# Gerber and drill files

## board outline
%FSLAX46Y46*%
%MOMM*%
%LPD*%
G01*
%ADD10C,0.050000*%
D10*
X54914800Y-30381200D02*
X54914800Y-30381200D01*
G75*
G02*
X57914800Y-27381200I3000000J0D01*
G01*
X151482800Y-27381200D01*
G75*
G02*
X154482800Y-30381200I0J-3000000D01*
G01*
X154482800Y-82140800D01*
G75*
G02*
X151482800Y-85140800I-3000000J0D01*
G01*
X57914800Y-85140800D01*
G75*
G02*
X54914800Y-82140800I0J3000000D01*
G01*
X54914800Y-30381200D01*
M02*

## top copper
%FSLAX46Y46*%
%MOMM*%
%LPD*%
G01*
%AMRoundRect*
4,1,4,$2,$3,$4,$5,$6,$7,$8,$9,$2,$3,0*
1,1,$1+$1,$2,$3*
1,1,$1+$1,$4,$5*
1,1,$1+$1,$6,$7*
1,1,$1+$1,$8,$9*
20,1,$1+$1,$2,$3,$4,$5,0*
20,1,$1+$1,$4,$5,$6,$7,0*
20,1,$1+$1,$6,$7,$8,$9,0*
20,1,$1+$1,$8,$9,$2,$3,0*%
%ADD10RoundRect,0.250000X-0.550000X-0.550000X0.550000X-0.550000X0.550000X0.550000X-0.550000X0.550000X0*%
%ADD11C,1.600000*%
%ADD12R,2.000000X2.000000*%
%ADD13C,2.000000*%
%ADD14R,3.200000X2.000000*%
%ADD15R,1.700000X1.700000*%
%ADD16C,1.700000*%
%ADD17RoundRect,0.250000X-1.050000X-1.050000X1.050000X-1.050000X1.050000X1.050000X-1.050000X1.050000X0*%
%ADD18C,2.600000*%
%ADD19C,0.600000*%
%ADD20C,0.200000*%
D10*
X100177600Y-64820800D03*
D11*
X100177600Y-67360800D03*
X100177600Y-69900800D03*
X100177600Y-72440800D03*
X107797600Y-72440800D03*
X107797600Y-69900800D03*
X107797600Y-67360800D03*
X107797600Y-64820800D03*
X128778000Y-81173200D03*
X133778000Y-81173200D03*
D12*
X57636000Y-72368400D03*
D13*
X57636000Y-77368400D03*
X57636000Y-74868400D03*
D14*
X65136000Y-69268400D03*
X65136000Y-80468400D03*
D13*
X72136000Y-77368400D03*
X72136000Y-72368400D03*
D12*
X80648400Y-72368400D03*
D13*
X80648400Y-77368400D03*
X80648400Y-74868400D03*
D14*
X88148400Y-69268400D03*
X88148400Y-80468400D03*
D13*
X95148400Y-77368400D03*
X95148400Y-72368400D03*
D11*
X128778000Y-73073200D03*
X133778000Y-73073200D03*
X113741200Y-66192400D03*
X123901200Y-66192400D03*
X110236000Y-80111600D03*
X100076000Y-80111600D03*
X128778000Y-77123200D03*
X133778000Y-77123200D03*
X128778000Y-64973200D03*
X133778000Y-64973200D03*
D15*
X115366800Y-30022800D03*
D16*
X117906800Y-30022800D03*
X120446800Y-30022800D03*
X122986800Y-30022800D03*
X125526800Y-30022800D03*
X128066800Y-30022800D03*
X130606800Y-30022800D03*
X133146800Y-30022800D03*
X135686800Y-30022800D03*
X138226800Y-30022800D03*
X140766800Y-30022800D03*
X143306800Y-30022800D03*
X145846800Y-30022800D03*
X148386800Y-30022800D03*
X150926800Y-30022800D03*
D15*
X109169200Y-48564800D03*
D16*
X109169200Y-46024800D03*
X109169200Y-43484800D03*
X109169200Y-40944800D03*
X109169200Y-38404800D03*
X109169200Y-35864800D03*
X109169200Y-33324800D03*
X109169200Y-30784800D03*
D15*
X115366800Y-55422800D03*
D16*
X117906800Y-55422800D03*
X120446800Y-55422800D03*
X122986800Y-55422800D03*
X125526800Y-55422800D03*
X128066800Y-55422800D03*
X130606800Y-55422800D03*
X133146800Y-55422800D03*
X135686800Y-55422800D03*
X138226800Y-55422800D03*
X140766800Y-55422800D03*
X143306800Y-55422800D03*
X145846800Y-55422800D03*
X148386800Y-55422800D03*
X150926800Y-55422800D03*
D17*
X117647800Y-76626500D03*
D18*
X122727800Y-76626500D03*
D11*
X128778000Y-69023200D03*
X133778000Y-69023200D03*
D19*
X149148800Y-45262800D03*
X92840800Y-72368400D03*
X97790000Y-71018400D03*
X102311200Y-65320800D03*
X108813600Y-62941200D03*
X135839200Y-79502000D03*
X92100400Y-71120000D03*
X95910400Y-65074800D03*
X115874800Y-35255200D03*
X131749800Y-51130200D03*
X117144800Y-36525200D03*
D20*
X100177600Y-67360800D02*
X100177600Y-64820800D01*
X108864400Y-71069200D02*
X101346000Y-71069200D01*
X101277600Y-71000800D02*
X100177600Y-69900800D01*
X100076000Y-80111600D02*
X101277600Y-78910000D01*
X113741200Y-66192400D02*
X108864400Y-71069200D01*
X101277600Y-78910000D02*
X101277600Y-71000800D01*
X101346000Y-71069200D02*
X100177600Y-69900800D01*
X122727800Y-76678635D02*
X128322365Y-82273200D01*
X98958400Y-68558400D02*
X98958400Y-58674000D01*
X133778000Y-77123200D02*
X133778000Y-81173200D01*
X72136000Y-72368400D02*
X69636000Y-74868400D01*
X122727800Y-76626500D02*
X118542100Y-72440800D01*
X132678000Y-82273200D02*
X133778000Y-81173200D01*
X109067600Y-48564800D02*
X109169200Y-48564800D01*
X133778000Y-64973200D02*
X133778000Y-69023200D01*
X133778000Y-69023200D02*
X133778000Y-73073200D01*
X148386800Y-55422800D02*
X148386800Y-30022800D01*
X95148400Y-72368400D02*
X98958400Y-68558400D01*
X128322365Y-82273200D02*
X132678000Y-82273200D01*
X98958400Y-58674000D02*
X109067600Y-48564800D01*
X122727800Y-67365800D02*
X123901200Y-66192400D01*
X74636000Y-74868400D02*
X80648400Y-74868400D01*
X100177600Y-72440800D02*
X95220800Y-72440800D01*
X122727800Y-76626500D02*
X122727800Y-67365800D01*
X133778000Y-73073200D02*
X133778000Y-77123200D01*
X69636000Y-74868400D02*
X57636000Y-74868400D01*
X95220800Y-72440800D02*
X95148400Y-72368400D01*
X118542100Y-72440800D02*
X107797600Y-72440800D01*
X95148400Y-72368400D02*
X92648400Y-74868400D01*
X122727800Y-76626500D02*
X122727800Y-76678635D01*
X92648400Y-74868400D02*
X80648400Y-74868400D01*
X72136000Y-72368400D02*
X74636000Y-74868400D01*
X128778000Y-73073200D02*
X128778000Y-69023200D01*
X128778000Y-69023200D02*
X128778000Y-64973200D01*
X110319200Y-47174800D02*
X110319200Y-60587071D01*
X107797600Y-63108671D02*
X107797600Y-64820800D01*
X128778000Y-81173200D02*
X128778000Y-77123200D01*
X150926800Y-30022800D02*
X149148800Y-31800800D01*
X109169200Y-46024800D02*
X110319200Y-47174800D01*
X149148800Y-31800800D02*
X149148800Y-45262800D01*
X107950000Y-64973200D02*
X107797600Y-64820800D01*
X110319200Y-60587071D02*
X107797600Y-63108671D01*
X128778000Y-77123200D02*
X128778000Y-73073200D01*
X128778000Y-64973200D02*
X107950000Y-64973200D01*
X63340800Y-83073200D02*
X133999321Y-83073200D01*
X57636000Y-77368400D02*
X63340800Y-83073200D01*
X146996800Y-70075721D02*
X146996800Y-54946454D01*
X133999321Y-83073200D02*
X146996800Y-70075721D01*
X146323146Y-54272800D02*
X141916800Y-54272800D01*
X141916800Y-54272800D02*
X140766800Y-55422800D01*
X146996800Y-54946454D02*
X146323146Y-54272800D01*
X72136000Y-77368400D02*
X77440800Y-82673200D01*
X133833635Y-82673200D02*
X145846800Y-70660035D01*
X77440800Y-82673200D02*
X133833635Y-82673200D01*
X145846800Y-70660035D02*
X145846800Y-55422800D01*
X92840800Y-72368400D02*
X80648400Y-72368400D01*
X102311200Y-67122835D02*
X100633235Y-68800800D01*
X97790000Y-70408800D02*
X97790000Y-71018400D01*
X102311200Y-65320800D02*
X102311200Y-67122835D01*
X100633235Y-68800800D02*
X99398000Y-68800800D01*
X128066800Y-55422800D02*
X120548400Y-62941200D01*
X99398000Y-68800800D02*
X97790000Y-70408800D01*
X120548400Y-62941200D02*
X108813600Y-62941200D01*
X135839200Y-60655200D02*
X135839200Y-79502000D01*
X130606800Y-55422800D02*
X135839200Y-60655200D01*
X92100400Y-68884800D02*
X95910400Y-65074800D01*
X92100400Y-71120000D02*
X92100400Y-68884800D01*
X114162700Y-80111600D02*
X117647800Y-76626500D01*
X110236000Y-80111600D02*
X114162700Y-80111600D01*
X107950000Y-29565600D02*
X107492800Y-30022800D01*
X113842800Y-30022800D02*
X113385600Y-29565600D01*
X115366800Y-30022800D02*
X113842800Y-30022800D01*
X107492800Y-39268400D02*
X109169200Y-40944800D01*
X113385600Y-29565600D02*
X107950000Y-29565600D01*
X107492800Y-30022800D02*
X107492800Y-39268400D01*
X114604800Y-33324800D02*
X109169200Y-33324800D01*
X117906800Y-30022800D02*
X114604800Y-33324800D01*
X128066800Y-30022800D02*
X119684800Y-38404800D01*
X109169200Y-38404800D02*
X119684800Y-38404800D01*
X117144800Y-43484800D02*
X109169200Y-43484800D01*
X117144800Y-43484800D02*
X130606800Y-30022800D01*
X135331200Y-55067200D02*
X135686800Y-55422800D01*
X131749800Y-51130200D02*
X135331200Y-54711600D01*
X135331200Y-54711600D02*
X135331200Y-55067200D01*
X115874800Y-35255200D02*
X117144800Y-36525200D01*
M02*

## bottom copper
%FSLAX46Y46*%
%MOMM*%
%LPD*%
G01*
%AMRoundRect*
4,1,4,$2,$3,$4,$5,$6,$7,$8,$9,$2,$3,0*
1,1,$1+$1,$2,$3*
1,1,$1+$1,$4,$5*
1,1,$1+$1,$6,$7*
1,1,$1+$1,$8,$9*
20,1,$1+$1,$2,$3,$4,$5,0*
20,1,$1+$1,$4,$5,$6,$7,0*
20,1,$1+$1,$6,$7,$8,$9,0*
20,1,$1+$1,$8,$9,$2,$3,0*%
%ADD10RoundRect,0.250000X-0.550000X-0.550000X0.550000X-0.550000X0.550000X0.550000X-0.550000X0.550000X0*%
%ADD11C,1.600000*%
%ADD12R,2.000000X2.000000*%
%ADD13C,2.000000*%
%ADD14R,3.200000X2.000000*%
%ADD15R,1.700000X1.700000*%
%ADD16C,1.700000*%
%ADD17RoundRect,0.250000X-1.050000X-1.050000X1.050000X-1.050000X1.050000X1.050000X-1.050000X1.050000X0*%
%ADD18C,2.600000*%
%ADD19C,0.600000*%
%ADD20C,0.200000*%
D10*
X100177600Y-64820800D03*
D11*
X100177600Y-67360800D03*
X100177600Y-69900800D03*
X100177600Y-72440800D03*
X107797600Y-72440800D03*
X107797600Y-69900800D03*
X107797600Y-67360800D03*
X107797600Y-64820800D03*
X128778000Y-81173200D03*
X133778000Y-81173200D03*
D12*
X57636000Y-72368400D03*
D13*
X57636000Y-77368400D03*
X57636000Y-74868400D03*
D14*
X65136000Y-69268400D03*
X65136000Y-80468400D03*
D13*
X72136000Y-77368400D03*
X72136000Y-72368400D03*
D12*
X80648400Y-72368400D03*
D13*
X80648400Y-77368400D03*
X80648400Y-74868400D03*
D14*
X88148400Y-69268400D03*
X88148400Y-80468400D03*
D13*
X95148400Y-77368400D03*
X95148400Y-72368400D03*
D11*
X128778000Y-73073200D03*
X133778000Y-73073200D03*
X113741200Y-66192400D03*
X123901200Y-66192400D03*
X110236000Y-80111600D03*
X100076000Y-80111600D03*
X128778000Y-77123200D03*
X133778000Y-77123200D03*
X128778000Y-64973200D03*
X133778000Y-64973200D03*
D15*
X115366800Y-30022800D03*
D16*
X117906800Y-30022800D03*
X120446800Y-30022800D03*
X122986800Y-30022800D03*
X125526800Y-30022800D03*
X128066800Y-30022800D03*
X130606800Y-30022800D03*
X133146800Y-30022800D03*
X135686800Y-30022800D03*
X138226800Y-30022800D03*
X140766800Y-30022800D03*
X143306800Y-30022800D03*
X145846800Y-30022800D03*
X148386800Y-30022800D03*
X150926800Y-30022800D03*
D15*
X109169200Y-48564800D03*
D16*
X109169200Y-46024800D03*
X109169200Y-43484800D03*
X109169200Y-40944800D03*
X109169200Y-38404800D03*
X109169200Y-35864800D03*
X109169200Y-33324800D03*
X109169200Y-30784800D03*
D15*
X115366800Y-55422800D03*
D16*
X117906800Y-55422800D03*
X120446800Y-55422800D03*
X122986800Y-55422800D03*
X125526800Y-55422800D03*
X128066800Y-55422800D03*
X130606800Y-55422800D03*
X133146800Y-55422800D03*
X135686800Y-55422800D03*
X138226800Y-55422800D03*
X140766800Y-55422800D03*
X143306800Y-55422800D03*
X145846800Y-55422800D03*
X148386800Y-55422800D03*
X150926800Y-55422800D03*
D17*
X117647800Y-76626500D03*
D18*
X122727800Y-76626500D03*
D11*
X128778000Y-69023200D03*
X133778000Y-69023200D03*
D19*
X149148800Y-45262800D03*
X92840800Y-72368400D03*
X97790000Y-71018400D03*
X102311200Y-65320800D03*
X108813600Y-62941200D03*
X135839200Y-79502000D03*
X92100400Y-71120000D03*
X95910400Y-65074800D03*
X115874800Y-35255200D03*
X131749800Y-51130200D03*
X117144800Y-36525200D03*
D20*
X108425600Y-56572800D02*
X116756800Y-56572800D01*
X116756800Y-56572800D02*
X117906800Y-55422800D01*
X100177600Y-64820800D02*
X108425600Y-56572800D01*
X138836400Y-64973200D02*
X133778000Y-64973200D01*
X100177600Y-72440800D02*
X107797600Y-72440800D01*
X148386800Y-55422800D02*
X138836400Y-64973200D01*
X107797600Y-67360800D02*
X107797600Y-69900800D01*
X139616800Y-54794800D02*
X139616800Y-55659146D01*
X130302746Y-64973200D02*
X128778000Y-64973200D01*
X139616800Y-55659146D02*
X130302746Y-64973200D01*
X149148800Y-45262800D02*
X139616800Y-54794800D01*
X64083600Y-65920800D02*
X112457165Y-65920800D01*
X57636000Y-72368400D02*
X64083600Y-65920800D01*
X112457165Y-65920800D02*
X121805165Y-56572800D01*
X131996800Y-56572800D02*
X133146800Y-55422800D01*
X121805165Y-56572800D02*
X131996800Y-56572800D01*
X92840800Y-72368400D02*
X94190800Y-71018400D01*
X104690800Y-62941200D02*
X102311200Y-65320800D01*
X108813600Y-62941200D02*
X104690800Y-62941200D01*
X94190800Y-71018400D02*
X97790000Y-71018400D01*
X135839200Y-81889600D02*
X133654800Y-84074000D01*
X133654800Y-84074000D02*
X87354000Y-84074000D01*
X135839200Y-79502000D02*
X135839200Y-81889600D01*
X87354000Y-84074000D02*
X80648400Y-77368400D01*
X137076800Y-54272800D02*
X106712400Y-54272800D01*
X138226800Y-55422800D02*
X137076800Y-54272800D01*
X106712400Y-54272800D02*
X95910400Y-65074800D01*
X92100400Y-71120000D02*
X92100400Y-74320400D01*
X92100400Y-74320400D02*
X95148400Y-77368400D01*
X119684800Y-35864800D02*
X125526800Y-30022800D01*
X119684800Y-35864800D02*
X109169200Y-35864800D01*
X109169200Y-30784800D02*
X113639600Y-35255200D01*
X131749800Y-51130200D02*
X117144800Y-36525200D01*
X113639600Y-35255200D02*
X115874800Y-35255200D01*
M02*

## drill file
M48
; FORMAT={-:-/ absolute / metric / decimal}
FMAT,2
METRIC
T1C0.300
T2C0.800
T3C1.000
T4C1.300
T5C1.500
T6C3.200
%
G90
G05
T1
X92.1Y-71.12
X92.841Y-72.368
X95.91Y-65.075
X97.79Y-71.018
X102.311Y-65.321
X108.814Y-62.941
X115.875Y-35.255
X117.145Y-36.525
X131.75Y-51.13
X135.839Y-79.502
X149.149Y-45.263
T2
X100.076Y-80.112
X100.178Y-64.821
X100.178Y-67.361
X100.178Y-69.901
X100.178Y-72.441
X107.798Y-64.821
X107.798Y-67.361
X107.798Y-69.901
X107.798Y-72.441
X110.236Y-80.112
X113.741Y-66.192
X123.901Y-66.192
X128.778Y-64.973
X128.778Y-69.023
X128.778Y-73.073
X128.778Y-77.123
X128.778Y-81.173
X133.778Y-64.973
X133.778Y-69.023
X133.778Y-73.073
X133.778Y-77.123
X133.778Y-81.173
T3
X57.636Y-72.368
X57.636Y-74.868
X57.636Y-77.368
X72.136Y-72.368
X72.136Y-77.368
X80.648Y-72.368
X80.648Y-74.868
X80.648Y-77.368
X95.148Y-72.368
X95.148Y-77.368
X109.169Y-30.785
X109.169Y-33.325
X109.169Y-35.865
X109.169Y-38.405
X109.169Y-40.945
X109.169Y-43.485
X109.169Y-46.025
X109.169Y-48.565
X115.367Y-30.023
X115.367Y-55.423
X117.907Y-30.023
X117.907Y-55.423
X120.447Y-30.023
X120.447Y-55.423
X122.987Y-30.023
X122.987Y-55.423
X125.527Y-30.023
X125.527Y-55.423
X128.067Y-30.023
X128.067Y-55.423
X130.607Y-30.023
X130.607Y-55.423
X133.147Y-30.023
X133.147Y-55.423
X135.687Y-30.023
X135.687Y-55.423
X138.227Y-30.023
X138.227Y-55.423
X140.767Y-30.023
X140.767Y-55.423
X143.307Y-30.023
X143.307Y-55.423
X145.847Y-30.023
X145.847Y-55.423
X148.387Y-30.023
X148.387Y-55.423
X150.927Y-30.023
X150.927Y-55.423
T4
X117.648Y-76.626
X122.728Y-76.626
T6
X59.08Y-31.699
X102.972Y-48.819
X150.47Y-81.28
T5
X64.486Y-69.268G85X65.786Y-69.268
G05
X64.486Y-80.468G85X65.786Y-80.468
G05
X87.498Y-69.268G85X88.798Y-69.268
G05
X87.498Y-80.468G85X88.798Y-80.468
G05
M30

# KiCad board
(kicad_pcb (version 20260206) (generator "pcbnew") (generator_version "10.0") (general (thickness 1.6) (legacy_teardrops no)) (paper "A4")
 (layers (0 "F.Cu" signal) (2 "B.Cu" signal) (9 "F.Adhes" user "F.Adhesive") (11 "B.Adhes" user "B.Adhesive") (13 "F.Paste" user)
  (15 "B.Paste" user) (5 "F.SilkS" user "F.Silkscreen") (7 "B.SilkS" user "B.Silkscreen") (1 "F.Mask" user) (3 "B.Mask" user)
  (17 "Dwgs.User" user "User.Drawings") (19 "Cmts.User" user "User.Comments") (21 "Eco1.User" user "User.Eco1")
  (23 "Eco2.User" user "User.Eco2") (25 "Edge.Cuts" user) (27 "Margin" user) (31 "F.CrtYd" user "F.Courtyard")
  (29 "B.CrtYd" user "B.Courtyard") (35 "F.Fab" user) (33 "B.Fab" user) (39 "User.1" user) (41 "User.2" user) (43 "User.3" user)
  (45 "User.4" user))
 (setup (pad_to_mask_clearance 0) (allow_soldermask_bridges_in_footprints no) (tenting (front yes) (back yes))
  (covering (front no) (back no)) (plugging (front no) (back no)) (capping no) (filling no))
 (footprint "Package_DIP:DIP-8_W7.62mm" (layer "F.Cu") (at 100.1776 64.8208)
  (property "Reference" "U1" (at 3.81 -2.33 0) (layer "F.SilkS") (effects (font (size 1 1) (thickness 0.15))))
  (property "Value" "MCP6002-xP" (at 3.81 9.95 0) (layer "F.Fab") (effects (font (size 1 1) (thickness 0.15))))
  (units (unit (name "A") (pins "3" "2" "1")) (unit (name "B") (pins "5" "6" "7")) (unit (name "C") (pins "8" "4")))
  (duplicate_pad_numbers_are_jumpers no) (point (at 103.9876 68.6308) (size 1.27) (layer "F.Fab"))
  (pad "1" thru_hole roundrect (at 0 0) (size 1.6 1.6) (drill 0.8) (layers "*.Cu" "*.Mask") (remove_unused_layers no)
   (roundrect_rratio 0.15625) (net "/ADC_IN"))
  (pad "2" thru_hole circle (at 0 2.54) (size 1.6 1.6) (drill 0.8) (layers "*.Cu" "*.Mask") (remove_unused_layers no) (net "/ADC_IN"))
  (pad "3" thru_hole circle (at 0 5.08) (size 1.6 1.6) (drill 0.8) (layers "*.Cu" "*.Mask") (remove_unused_layers no) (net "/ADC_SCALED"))
  (pad "4" thru_hole circle (at 0 7.62) (size 1.6 1.6) (drill 0.8) (layers "*.Cu" "*.Mask") (remove_unused_layers no) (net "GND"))
  (pad "5" thru_hole circle (at 7.62 7.62) (size 1.6 1.6) (drill 0.8) (layers "*.Cu" "*.Mask") (remove_unused_layers no) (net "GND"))
  (pad "6" thru_hole circle (at 7.62 5.08) (size 1.6 1.6) (drill 0.8) (layers "*.Cu" "*.Mask") (remove_unused_layers no) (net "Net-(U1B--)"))
  (pad "7" thru_hole circle (at 7.62 2.54) (size 1.6 1.6) (drill 0.8) (layers "*.Cu" "*.Mask") (remove_unused_layers no) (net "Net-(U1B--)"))
  (pad "8" thru_hole circle (at 7.62 0) (size 1.6 1.6) (drill 0.8) (layers "*.Cu" "*.Mask") (remove_unused_layers no) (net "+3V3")))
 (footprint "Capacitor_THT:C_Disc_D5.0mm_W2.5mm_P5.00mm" (layer "F.Cu") (at 128.778 81.1732)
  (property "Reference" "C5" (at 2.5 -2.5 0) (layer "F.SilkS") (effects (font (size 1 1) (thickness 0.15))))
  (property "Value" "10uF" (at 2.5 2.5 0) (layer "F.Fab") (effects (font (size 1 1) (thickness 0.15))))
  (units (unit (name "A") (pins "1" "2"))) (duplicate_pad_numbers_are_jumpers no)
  (pad "1" thru_hole circle (at 0 0) (size 1.6 1.6) (drill 0.8) (layers "*.Cu" "*.Mask") (remove_unused_layers no) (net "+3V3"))
  (pad "2" thru_hole circle (at 5 0) (size 1.6 1.6) (drill 0.8) (layers "*.Cu" "*.Mask") (remove_unused_layers no) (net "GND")))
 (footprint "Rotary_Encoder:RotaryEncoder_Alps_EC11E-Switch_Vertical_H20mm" (layer "F.Cu") (at 57.636 72.3684)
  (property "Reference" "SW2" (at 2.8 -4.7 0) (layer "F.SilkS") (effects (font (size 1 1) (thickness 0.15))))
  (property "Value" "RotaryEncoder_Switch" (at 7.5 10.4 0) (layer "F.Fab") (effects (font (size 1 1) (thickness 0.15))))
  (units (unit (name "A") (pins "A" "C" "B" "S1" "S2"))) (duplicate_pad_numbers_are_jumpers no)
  (pad "A" thru_hole rect (at 0 0) (size 2 2) (drill 1) (layers "*.Cu" "*.Mask") (remove_unused_layers no) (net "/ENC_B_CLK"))
  (pad "B" thru_hole circle (at 0 5) (size 2 2) (drill 1) (layers "*.Cu" "*.Mask") (remove_unused_layers no) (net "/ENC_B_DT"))
  (pad "C" thru_hole circle (at 0 2.5) (size 2 2) (drill 1) (layers "*.Cu" "*.Mask") (remove_unused_layers no) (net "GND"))
  (pad "MP" thru_hole rect (at 7.5 -3.1) (size 3.2 2) (drill oval 2.8 1.5) (layers "*.Cu" "*.Mask") (remove_unused_layers no))
  (pad "MP" thru_hole rect (at 7.5 8.1) (size 3.2 2) (drill oval 2.8 1.5) (layers "*.Cu" "*.Mask") (remove_unused_layers no))
  (pad "S1" thru_hole circle (at 14.5 5) (size 2 2) (drill 1) (layers "*.Cu" "*.Mask") (remove_unused_layers no) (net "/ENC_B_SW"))
  (pad "S2" thru_hole circle (at 14.5 0) (size 2 2) (drill 1) (layers "*.Cu" "*.Mask") (remove_unused_layers no) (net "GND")))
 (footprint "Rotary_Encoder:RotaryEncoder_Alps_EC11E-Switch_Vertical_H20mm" (layer "F.Cu") (at 80.6484 72.3684)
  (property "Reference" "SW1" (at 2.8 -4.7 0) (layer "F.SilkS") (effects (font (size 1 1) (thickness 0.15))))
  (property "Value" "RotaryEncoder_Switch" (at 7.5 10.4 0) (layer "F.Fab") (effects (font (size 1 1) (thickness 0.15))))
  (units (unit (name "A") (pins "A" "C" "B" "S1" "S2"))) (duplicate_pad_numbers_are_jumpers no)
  (pad "A" thru_hole rect (at 0 0) (size 2 2) (drill 1) (layers "*.Cu" "*.Mask") (remove_unused_layers no) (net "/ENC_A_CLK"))
  (pad "B" thru_hole circle (at 0 5) (size 2 2) (drill 1) (layers "*.Cu" "*.Mask") (remove_unused_layers no) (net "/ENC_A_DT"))
  (pad "C" thru_hole circle (at 0 2.5) (size 2 2) (drill 1) (layers "*.Cu" "*.Mask") (remove_unused_layers no) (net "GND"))
  (pad "MP" thru_hole rect (at 7.5 -3.1) (size 3.2 2) (drill oval 2.8 1.5) (layers "*.Cu" "*.Mask") (remove_unused_layers no))
  (pad "MP" thru_hole rect (at 7.5 8.1) (size 3.2 2) (drill oval 2.8 1.5) (layers "*.Cu" "*.Mask") (remove_unused_layers no))
  (pad "S1" thru_hole circle (at 14.5 5) (size 2 2) (drill 1) (layers "*.Cu" "*.Mask") (remove_unused_layers no) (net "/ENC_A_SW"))
  (pad "S2" thru_hole circle (at 14.5 0) (size 2 2) (drill 1) (layers "*.Cu" "*.Mask") (remove_unused_layers no) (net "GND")))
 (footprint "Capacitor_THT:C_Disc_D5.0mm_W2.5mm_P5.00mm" (layer "F.Cu") (at 128.778 73.0732)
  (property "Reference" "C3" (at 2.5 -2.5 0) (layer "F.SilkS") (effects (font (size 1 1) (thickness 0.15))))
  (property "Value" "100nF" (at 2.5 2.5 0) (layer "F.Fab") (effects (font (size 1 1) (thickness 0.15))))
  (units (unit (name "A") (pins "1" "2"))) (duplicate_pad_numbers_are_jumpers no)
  (pad "1" thru_hole circle (at 0 0) (size 1.6 1.6) (drill 0.8) (layers "*.Cu" "*.Mask") (remove_unused_layers no) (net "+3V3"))
  (pad "2" thru_hole circle (at 5 0) (size 1.6 1.6) (drill 0.8) (layers "*.Cu" "*.Mask") (remove_unused_layers no) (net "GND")))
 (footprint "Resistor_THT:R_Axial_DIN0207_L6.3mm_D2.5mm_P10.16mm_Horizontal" (layer "F.Cu") (at 113.7412 66.1924)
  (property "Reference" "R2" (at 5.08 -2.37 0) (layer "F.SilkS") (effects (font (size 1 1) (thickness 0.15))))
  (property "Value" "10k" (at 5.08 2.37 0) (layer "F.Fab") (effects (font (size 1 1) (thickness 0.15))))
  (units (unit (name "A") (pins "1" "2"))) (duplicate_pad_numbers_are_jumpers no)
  (pad "1" thru_hole circle (at 0 0) (size 1.6 1.6) (drill 0.8) (layers "*.Cu" "*.Mask") (remove_unused_layers no) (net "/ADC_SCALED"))
  (pad "2" thru_hole circle (at 10.16 0) (size 1.6 1.6) (drill 0.8) (layers "*.Cu" "*.Mask") (remove_unused_layers no) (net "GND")))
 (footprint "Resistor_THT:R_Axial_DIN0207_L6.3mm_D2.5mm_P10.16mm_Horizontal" (layer "F.Cu") (at 110.236 80.1116 180)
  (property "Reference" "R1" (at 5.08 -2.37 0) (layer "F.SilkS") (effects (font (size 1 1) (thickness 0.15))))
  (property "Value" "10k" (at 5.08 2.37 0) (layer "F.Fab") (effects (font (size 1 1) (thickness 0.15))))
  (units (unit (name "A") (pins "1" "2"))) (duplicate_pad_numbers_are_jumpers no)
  (pad "1" thru_hole circle (at 0 0 180) (size 1.6 1.6) (drill 0.8) (layers "*.Cu" "*.Mask") (remove_unused_layers no) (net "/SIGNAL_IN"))
  (pad "2" thru_hole circle (at 10.16 0 180) (size 1.6 1.6) (drill 0.8) (layers "*.Cu" "*.Mask") (remove_unused_layers no)
   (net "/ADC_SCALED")))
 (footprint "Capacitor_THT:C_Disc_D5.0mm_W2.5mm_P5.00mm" (layer "F.Cu") (at 128.778 77.1232)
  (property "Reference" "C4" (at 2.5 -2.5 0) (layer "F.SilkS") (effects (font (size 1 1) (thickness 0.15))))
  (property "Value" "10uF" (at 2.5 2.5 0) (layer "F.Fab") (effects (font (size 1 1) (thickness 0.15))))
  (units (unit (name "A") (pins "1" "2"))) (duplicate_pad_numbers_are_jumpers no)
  (pad "1" thru_hole circle (at 0 0) (size 1.6 1.6) (drill 0.8) (layers "*.Cu" "*.Mask") (remove_unused_layers no) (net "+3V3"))
  (pad "2" thru_hole circle (at 5 0) (size 1.6 1.6) (drill 0.8) (layers "*.Cu" "*.Mask") (remove_unused_layers no) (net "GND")))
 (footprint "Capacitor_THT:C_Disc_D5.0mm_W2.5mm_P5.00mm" (layer "F.Cu") (at 128.778 64.9732)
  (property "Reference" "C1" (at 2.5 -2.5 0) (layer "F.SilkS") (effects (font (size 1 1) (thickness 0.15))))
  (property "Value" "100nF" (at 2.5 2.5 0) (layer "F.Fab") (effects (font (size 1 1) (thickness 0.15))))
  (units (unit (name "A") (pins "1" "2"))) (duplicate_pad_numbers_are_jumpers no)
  (pad "1" thru_hole circle (at 0 0) (size 1.6 1.6) (drill 0.8) (layers "*.Cu" "*.Mask") (remove_unused_layers no) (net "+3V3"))
  (pad "2" thru_hole circle (at 5 0) (size 1.6 1.6) (drill 0.8) (layers "*.Cu" "*.Mask") (remove_unused_layers no) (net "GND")))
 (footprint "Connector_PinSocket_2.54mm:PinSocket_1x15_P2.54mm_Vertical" (layer "F.Cu") (at 115.3668 30.0228 90)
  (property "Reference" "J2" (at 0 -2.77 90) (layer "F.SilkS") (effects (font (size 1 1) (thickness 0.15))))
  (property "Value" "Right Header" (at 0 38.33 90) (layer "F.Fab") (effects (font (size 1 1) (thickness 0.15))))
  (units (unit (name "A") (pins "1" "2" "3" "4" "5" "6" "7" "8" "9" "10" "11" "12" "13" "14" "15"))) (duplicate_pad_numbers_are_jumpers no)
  (pad "1" thru_hole rect (at 0 0 90) (size 1.7 1.7) (drill 1) (layers "*.Cu" "*.Mask") (remove_unused_layers no) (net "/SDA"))
  (pad "2" thru_hole circle (at 0 2.54 90) (size 1.7 1.7) (drill 1) (layers "*.Cu" "*.Mask") (remove_unused_layers no) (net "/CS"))
  (pad "3" thru_hole circle (at 0 5.08 90) (size 1.7 1.7) (drill 1) (layers "*.Cu" "*.Mask") (remove_unused_layers no) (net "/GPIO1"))
  (pad "4" thru_hole circle (at 0 7.62 90) (size 1.7 1.7) (drill 1) (layers "*.Cu" "*.Mask") (remove_unused_layers no) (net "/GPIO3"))
  (pad "5" thru_hole circle (at 0 10.16 90) (size 1.7 1.7) (drill 1) (layers "*.Cu" "*.Mask") (remove_unused_layers no) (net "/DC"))
  (pad "6" thru_hole circle (at 0 12.7 90) (size 1.7 1.7) (drill 1) (layers "*.Cu" "*.Mask") (remove_unused_layers no) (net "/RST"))
  (pad "7" thru_hole circle (at 0 15.24 90) (size 1.7 1.7) (drill 1) (layers "*.Cu" "*.Mask") (remove_unused_layers no) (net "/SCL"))
  (pad "8" thru_hole circle (at 0 17.78 90) (size 1.7 1.7) (drill 1) (layers "*.Cu" "*.Mask") (remove_unused_layers no) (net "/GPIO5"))
  (pad "9" thru_hole circle (at 0 20.32 90) (size 1.7 1.7) (drill 1) (layers "*.Cu" "*.Mask") (remove_unused_layers no) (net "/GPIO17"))
  (pad "10" thru_hole circle (at 0 22.86 90) (size 1.7 1.7) (drill 1) (layers "*.Cu" "*.Mask") (remove_unused_layers no) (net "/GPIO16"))
  (pad "11" thru_hole circle (at 0 25.4 90) (size 1.7 1.7) (drill 1) (layers "*.Cu" "*.Mask") (remove_unused_layers no) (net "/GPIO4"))
  (pad "12" thru_hole circle (at 0 27.94 90) (size 1.7 1.7) (drill 1) (layers "*.Cu" "*.Mask") (remove_unused_layers no) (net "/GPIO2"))
  (pad "13" thru_hole circle (at 0 30.48 90) (size 1.7 1.7) (drill 1) (layers "*.Cu" "*.Mask") (remove_unused_layers no) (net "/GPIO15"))
  (pad "14" thru_hole circle (at 0 33.02 90) (size 1.7 1.7) (drill 1) (layers "*.Cu" "*.Mask") (remove_unused_layers no) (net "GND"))
  (pad "15" thru_hole circle (at 0 35.56 90) (size 1.7 1.7) (drill 1) (layers "*.Cu" "*.Mask") (remove_unused_layers no) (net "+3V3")))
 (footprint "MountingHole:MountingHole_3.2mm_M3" (layer "F.Cu") (at 150.4696 81.28)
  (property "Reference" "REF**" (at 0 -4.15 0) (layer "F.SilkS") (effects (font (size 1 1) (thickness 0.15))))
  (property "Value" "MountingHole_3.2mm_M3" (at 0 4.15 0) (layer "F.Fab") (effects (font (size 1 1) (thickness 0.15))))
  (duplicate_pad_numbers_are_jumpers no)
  (pad "" np_thru_hole circle (at 0 0) (size 3.2 3.2) (drill 3.2) (layers "*.Cu" "*.Mask")))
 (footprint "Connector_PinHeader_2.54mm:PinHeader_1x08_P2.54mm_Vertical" (layer "F.Cu") (at 109.1692 48.5648 180)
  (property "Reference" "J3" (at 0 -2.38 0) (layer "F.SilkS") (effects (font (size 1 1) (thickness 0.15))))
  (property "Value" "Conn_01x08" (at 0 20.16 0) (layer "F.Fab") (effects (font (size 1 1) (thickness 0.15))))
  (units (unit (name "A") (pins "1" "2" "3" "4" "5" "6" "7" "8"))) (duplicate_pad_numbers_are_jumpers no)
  (pad "1" thru_hole rect (at 0 0 180) (size 1.7 1.7) (drill 1) (layers "*.Cu" "*.Mask") (remove_unused_layers no) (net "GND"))
  (pad "2" thru_hole circle (at 0 2.54 180) (size 1.7 1.7) (drill 1) (layers "*.Cu" "*.Mask") (remove_unused_layers no) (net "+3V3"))
  (pad "3" thru_hole circle (at 0 5.08 180) (size 1.7 1.7) (drill 1) (layers "*.Cu" "*.Mask") (remove_unused_layers no) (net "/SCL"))
  (pad "4" thru_hole circle (at 0 7.62 180) (size 1.7 1.7) (drill 1) (layers "*.Cu" "*.Mask") (remove_unused_layers no) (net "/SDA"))
  (pad "5" thru_hole circle (at 0 10.16 180) (size 1.7 1.7) (drill 1) (layers "*.Cu" "*.Mask") (remove_unused_layers no) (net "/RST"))
  (pad "6" thru_hole circle (at 0 12.7 180) (size 1.7 1.7) (drill 1) (layers "*.Cu" "*.Mask") (remove_unused_layers no) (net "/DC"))
  (pad "7" thru_hole circle (at 0 15.24 180) (size 1.7 1.7) (drill 1) (layers "*.Cu" "*.Mask") (remove_unused_layers no) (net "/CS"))
  (pad "8" thru_hole circle (at 0 17.78 180) (size 1.7 1.7) (drill 1) (layers "*.Cu" "*.Mask") (remove_unused_layers no) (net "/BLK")))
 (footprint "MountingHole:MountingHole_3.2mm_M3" (layer "F.Cu") (at 102.9716 48.8188)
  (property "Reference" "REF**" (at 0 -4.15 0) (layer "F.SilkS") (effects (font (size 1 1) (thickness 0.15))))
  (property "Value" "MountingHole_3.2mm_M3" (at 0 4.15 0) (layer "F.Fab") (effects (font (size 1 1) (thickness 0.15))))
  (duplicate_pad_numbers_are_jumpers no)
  (pad "" np_thru_hole circle (at 0 0) (size 3.2 3.2) (drill 3.2) (layers "*.Cu" "*.Mask")))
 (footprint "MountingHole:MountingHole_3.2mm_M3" (layer "F.Cu") (at 59.0804 31.6992)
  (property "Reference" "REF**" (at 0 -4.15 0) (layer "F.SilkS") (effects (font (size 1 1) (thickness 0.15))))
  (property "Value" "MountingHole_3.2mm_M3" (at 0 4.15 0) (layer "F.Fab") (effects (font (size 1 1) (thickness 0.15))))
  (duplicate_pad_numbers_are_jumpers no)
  (pad "" np_thru_hole circle (at 0 0) (size 3.2 3.2) (drill 3.2) (layers "*.Cu" "*.Mask")))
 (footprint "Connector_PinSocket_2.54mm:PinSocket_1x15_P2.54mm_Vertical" (layer "F.Cu") (at 115.3668 55.4228 90)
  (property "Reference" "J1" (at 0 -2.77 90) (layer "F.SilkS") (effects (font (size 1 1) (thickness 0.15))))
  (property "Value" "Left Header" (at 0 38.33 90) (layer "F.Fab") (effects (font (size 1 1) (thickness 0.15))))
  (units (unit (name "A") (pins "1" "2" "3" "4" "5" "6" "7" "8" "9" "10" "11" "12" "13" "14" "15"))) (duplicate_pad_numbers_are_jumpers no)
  (pad "1" thru_hole rect (at 0 0 90) (size 1.7 1.7) (drill 1) (layers "*.Cu" "*.Mask") (remove_unused_layers no) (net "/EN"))
  (pad "2" thru_hole circle (at 0 2.54 90) (size 1.7 1.7) (drill 1) (layers "*.Cu" "*.Mask") (remove_unused_layers no) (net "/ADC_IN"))
  (pad "3" thru_hole circle (at 0 5.08 90) (size 1.7 1.7) (drill 1) (layers "*.Cu" "*.Mask") (remove_unused_layers no) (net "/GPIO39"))
  (pad "4" thru_hole circle (at 0 7.62 90) (size 1.7 1.7) (drill 1) (layers "*.Cu" "*.Mask") (remove_unused_layers no) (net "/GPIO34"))
  (pad "5" thru_hole circle (at 0 10.16 90) (size 1.7 1.7) (drill 1) (layers "*.Cu" "*.Mask") (remove_unused_layers no) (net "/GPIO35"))
  (pad "6" thru_hole circle (at 0 12.7 90) (size 1.7 1.7) (drill 1) (layers "*.Cu" "*.Mask") (remove_unused_layers no) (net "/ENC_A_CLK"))
  (pad "7" thru_hole circle (at 0 15.24 90) (size 1.7 1.7) (drill 1) (layers "*.Cu" "*.Mask") (remove_unused_layers no) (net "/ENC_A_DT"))
  (pad "8" thru_hole circle (at 0 17.78 90) (size 1.7 1.7) (drill 1) (layers "*.Cu" "*.Mask") (remove_unused_layers no) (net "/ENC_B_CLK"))
  (pad "9" thru_hole circle (at 0 20.32 90) (size 1.7 1.7) (drill 1) (layers "*.Cu" "*.Mask") (remove_unused_layers no) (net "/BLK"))
  (pad "10" thru_hole circle (at 0 22.86 90) (size 1.7 1.7) (drill 1) (layers "*.Cu" "*.Mask") (remove_unused_layers no) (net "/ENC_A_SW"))
  (pad "11" thru_hole circle (at 0 25.4 90) (size 1.7 1.7) (drill 1) (layers "*.Cu" "*.Mask") (remove_unused_layers no) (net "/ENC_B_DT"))
  (pad "12" thru_hole circle (at 0 27.94 90) (size 1.7 1.7) (drill 1) (layers "*.Cu" "*.Mask") (remove_unused_layers no) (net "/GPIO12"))
  (pad "13" thru_hole circle (at 0 30.48 90) (size 1.7 1.7) (drill 1) (layers "*.Cu" "*.Mask") (remove_unused_layers no) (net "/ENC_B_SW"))
  (pad "14" thru_hole circle (at 0 33.02 90) (size 1.7 1.7) (drill 1) (layers "*.Cu" "*.Mask") (remove_unused_layers no) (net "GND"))
  (pad "15" thru_hole circle (at 0 35.56 90) (size 1.7 1.7) (drill 1) (layers "*.Cu" "*.Mask") (remove_unused_layers no) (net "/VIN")))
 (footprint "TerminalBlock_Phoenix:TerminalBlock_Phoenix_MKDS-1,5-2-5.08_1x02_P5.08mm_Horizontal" (layer "F.Cu") (at 117.6478 76.6265)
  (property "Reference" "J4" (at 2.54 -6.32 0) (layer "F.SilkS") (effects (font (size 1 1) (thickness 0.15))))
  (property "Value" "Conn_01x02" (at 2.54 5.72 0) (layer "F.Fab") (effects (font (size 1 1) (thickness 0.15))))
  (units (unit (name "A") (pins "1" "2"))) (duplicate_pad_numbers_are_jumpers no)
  (pad "1" thru_hole roundrect (at 0 0) (size 2.6 2.6) (drill 1.3) (layers "*.Cu" "*.Mask") (remove_unused_layers no)
   (roundrect_rratio 0.096154) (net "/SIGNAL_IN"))
  (pad "2" thru_hole circle (at 5.08 0) (size 2.6 2.6) (drill 1.3) (layers "*.Cu" "*.Mask") (remove_unused_layers no) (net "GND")))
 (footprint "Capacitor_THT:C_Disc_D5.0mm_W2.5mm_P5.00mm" (layer "F.Cu") (at 128.778 69.0232)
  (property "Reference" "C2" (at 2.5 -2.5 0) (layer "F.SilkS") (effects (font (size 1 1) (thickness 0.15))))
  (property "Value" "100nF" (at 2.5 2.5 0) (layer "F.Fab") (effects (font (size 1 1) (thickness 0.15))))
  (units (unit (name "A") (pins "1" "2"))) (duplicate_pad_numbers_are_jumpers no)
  (pad "1" thru_hole circle (at 0 0) (size 1.6 1.6) (drill 0.8) (layers "*.Cu" "*.Mask") (remove_unused_layers no) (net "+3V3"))
  (pad "2" thru_hole circle (at 5 0) (size 1.6 1.6) (drill 0.8) (layers "*.Cu" "*.Mask") (remove_unused_layers no) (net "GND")))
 (gr_rect (start 54.9148 27.3812) (end 154.4828 85.1408) (radius 3) (stroke (width 0.05) (type solid)) (fill no) (layer "Edge.Cuts"))
 (segment (start 100.1776 67.3608) (end 100.1776 64.8208) (width 0.2) (layer "F.Cu") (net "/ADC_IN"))
 (segment (start 108.4256 56.5728) (end 116.7568 56.5728) (width 0.2) (layer "B.Cu") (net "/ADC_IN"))
 (segment (start 116.7568 56.5728) (end 117.9068 55.4228) (width 0.2) (layer "B.Cu") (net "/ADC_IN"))
 (segment (start 100.1776 64.8208) (end 108.4256 56.5728) (width 0.2) (layer "B.Cu") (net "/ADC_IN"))
 (segment (start 108.8644 71.0692) (end 101.346 71.0692) (width 0.2) (layer "F.Cu") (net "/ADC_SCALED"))
 (segment (start 101.2776 71.0008) (end 100.1776 69.9008) (width 0.2) (layer "F.Cu") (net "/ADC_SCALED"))
 (segment (start 100.076 80.1116) (end 101.2776 78.91) (width 0.2) (layer "F.Cu") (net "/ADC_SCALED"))
 (segment (start 113.7412 66.1924) (end 108.8644 71.0692) (width 0.2) (layer "F.Cu") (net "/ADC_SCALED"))
 (segment (start 101.2776 78.91) (end 101.2776 71.0008) (width 0.2) (layer "F.Cu") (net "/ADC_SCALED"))
 (segment (start 101.346 71.0692) (end 100.1776 69.9008) (width 0.2) (layer "F.Cu") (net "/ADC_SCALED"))
 (segment (start 122.7278 76.678635) (end 128.322365 82.2732) (width 0.2) (layer "F.Cu") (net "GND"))
 (segment (start 98.9584 68.5584) (end 98.9584 58.674) (width 0.2) (layer "F.Cu") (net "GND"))
 (segment (start 133.778 77.1232) (end 133.778 81.1732) (width 0.2) (layer "F.Cu") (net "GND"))
 (segment (start 72.136 72.3684) (end 69.636 74.8684) (width 0.2) (layer "F.Cu") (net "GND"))
 (segment (start 122.7278 76.6265) (end 118.5421 72.4408) (width 0.2) (layer "F.Cu") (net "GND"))
 (segment (start 132.678 82.2732) (end 133.778 81.1732) (width 0.2) (layer "F.Cu") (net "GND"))
 (segment (start 109.0676 48.5648) (end 109.1692 48.5648) (width 0.2) (layer "F.Cu") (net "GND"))
 (segment (start 133.778 64.9732) (end 133.778 69.0232) (width 0.2) (layer "F.Cu") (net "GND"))
 (segment (start 133.778 69.0232) (end 133.778 73.0732) (width 0.2) (layer "F.Cu") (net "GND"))
 (segment (start 148.3868 55.4228) (end 148.3868 30.0228) (width 0.2) (layer "F.Cu") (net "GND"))
 (segment (start 95.1484 72.3684) (end 98.9584 68.5584) (width 0.2) (layer "F.Cu") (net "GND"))
 (segment (start 128.322365 82.2732) (end 132.678 82.2732) (width 0.2) (layer "F.Cu") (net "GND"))
 (segment (start 98.9584 58.674) (end 109.0676 48.5648) (width 0.2) (layer "F.Cu") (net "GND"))
 (segment (start 122.7278 67.3658) (end 123.9012 66.1924) (width 0.2) (layer "F.Cu") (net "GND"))
 (segment (start 74.636 74.8684) (end 80.6484 74.8684) (width 0.2) (layer "F.Cu") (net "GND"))
 (segment (start 100.1776 72.4408) (end 95.2208 72.4408) (width 0.2) (layer "F.Cu") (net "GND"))
 (segment (start 122.7278 76.6265) (end 122.7278 67.3658) (width 0.2) (layer "F.Cu") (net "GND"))
 (segment (start 133.778 73.0732) (end 133.778 77.1232) (width 0.2) (layer "F.Cu") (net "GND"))
 (segment (start 69.636 74.8684) (end 57.636 74.8684) (width 0.2) (layer "F.Cu") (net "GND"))
 (segment (start 95.2208 72.4408) (end 95.1484 72.3684) (width 0.2) (layer "F.Cu") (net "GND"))
 (segment (start 118.5421 72.4408) (end 107.7976 72.4408) (width 0.2) (layer "F.Cu") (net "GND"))
 (segment (start 95.1484 72.3684) (end 92.6484 74.8684) (width 0.2) (layer "F.Cu") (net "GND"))
 (segment (start 122.7278 76.6265) (end 122.7278 76.678635) (width 0.2) (layer "F.Cu") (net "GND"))
 (segment (start 92.6484 74.8684) (end 80.6484 74.8684) (width 0.2) (layer "F.Cu") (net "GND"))
 (segment (start 72.136 72.3684) (end 74.636 74.8684) (width 0.2) (layer "F.Cu") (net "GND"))
 (segment (start 138.8364 64.9732) (end 133.778 64.9732) (width 0.2) (layer "B.Cu") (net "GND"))
 (segment (start 100.1776 72.4408) (end 107.7976 72.4408) (width 0.2) (layer "B.Cu") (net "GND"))
 (segment (start 148.3868 55.4228) (end 138.8364 64.9732) (width 0.2) (layer "B.Cu") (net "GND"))
 (segment (start 107.7976 67.3608) (end 107.7976 69.9008) (width 0.2) (layer "B.Cu") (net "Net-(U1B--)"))
 (segment (start 128.778 73.0732) (end 128.778 69.0232) (width 0.2) (layer "F.Cu") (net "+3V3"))
 (segment (start 128.778 69.0232) (end 128.778 64.9732) (width 0.2) (layer "F.Cu") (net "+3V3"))
 (segment (start 110.3192 47.1748) (end 110.3192 60.587071) (width 0.2) (layer "F.Cu") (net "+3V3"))
 (segment (start 107.7976 63.108671) (end 107.7976 64.8208) (width 0.2) (layer "F.Cu") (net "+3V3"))
 (segment (start 128.778 81.1732) (end 128.778 77.1232) (width 0.2) (layer "F.Cu") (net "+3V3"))
 (segment (start 150.9268 30.0228) (end 149.1488 31.8008) (width 0.2) (layer "F.Cu") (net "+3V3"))
 (segment (start 109.1692 46.0248) (end 110.3192 47.1748) (width 0.2) (layer "F.Cu") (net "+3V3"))
 (segment (start 149.1488 31.8008) (end 149.1488 45.2628) (width 0.2) (layer "F.Cu") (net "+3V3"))
 (segment (start 107.95 64.9732) (end 107.7976 64.8208) (width 0.2) (layer "F.Cu") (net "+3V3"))
 (segment (start 110.3192 60.587071) (end 107.7976 63.108671) (width 0.2) (layer "F.Cu") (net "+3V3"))
 (segment (start 128.778 77.1232) (end 128.778 73.0732) (width 0.2) (layer "F.Cu") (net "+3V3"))
 (segment (start 128.778 64.9732) (end 107.95 64.9732) (width 0.2) (layer "F.Cu") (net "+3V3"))
 (via (at 149.1488 45.2628) (size 0.6) (drill 0.3) (layers "F.Cu" "B.Cu") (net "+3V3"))
 (segment (start 139.6168 54.7948) (end 139.6168 55.659146) (width 0.2) (layer "B.Cu") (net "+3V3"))
 (segment (start 130.302746 64.9732) (end 128.778 64.9732) (width 0.2) (layer "B.Cu") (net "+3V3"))
 (segment (start 139.6168 55.659146) (end 130.302746 64.9732) (width 0.2) (layer "B.Cu") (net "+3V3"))
 (segment (start 149.1488 45.2628) (end 139.6168 54.7948) (width 0.2) (layer "B.Cu") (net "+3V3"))
 (segment (start 64.0836 65.9208) (end 112.457165 65.9208) (width 0.2) (layer "B.Cu") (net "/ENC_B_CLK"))
 (segment (start 57.636 72.3684) (end 64.0836 65.9208) (width 0.2) (layer "B.Cu") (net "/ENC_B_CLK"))
 (segment (start 112.457165 65.9208) (end 121.805165 56.5728) (width 0.2) (layer "B.Cu") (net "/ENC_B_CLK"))
 (segment (start 131.9968 56.5728) (end 133.1468 55.4228) (width 0.2) (layer "B.Cu") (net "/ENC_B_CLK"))
 (segment (start 121.805165 56.5728) (end 131.9968 56.5728) (width 0.2) (layer "B.Cu") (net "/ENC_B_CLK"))
 (segment (start 63.3408 83.0732) (end 133.999321 83.0732) (width 0.2) (layer "F.Cu") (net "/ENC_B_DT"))
 (segment (start 57.636 77.3684) (end 63.3408 83.0732) (width 0.2) (layer "F.Cu") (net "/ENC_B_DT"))
 (segment (start 146.9968 70.075721) (end 146.9968 54.946454) (width 0.2) (layer "F.Cu") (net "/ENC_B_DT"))
 (segment (start 133.999321 83.0732) (end 146.9968 70.075721) (width 0.2) (layer "F.Cu") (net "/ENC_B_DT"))
 (segment (start 146.323146 54.2728) (end 141.9168 54.2728) (width 0.2) (layer "F.Cu") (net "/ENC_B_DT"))
 (segment (start 141.9168 54.2728) (end 140.7668 55.4228) (width 0.2) (layer "F.Cu") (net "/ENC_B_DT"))
 (segment (start 146.9968 54.946454) (end 146.323146 54.2728) (width 0.2) (layer "F.Cu") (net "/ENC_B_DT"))
 (segment (start 72.136 77.3684) (end 77.4408 82.6732) (width 0.2) (layer "F.Cu") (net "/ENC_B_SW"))
 (segment (start 133.833635 82.6732) (end 145.8468 70.660035) (width 0.2) (layer "F.Cu") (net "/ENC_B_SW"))
 (segment (start 77.4408 82.6732) (end 133.833635 82.6732) (width 0.2) (layer "F.Cu") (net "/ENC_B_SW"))
 (segment (start 145.8468 70.660035) (end 145.8468 55.4228) (width 0.2) (layer "F.Cu") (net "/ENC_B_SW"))
 (segment (start 92.8408 72.3684) (end 80.6484 72.3684) (width 0.2) (layer "F.Cu") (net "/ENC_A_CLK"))
 (segment (start 102.3112 67.122835) (end 100.633235 68.8008) (width 0.2) (layer "F.Cu") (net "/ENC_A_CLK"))
 (segment (start 97.79 70.4088) (end 97.79 71.0184) (width 0.2) (layer "F.Cu") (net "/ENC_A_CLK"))
 (segment (start 102.3112 65.3208) (end 102.3112 67.122835) (width 0.2) (layer "F.Cu") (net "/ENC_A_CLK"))
 (segment (start 100.633235 68.8008) (end 99.398 68.8008) (width 0.2) (layer "F.Cu") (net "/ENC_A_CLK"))
 (segment (start 128.0668 55.4228) (end 120.5484 62.9412) (width 0.2) (layer "F.Cu") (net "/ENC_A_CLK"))
 (segment (start 99.398 68.8008) (end 97.79 70.4088) (width 0.2) (layer "F.Cu") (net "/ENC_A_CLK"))
 (segment (start 120.5484 62.9412) (end 108.8136 62.9412) (width 0.2) (layer "F.Cu") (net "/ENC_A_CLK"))
 (via (at 92.8408 72.3684) (size 0.6) (drill 0.3) (layers "F.Cu" "B.Cu") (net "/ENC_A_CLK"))
 (via (at 97.79 71.0184) (size 0.6) (drill 0.3) (layers "F.Cu" "B.Cu") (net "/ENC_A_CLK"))
 (via (at 102.3112 65.3208) (size 0.6) (drill 0.3) (layers "F.Cu" "B.Cu") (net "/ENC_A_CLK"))
 (via (at 108.8136 62.9412) (size 0.6) (drill 0.3) (layers "F.Cu" "B.Cu") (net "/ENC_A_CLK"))
 (segment (start 92.8408 72.3684) (end 94.1908 71.0184) (width 0.2) (layer "B.Cu") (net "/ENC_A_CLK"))
 (segment (start 104.6908 62.9412) (end 102.3112 65.3208) (width 0.2) (layer "B.Cu") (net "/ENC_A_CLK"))
 (segment (start 108.8136 62.9412) (end 104.6908 62.9412) (width 0.2) (layer "B.Cu") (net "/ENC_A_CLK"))
 (segment (start 94.1908 71.0184) (end 97.79 71.0184) (width 0.2) (layer "B.Cu") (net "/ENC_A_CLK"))
 (segment (start 135.8392 60.6552) (end 135.8392 79.502) (width 0.2) (layer "F.Cu") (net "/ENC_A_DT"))
 (segment (start 130.6068 55.4228) (end 135.8392 60.6552) (width 0.2) (layer "F.Cu") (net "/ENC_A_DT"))
 (via (at 135.8392 79.502) (size 0.6) (drill 0.3) (layers "F.Cu" "B.Cu") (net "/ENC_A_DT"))
 (segment (start 135.8392 81.8896) (end 133.6548 84.074) (width 0.2) (layer "B.Cu") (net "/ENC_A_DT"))
 (segment (start 133.6548 84.074) (end 87.354 84.074) (width 0.2) (layer "B.Cu") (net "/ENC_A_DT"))
 (segment (start 135.8392 79.502) (end 135.8392 81.8896) (width 0.2) (layer "B.Cu") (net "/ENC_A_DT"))
 (segment (start 87.354 84.074) (end 80.6484 77.3684) (width 0.2) (layer "B.Cu") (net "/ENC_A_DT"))
 (segment (start 92.1004 68.8848) (end 95.9104 65.0748) (width 0.2) (layer "F.Cu") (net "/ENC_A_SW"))
 (segment (start 92.1004 71.12) (end 92.1004 68.8848) (width 0.2) (layer "F.Cu") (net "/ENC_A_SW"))
 (via (at 92.1004 71.12) (size 0.6) (drill 0.3) (layers "F.Cu" "B.Cu") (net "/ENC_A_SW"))
 (via (at 95.9104 65.0748) (size 0.6) (drill 0.3) (layers "F.Cu" "B.Cu") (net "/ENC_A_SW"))
 (segment (start 137.0768 54.2728) (end 106.7124 54.2728) (width 0.2) (layer "B.Cu") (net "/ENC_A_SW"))
 (segment (start 138.2268 55.4228) (end 137.0768 54.2728) (width 0.2) (layer "B.Cu") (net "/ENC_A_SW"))
 (segment (start 106.7124 54.2728) (end 95.9104 65.0748) (width 0.2) (layer "B.Cu") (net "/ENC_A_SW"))
 (segment (start 92.1004 71.12) (end 92.1004 74.3204) (width 0.2) (layer "B.Cu") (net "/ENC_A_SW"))
 (segment (start 92.1004 74.3204) (end 95.1484 77.3684) (width 0.2) (layer "B.Cu") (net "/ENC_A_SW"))
 (segment (start 114.1627 80.1116) (end 117.6478 76.6265) (width 0.2) (layer "F.Cu") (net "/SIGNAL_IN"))
 (segment (start 110.236 80.1116) (end 114.1627 80.1116) (width 0.2) (layer "F.Cu") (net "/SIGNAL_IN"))
 (segment (start 107.95 29.5656) (end 107.4928 30.0228) (width 0.2) (layer "F.Cu") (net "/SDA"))
 (segment (start 113.8428 30.0228) (end 113.3856 29.5656) (width 0.2) (layer "F.Cu") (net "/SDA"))
 (segment (start 115.3668 30.0228) (end 113.8428 30.0228) (width 0.2) (layer "F.Cu") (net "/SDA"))
 (segment (start 107.4928 39.2684) (end 109.1692 40.9448) (width 0.2) (layer "F.Cu") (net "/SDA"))
 (segment (start 113.3856 29.5656) (end 107.95 29.5656) (width 0.2) (layer "F.Cu") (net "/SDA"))
 (segment (start 107.4928 30.0228) (end 107.4928 39.2684) (width 0.2) (layer "F.Cu") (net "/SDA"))
 (segment (start 114.6048 33.3248) (end 109.1692 33.3248) (width 0.2) (layer "F.Cu") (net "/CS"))
 (segment (start 117.9068 30.0228) (end 114.6048 33.3248) (width 0.2) (layer "F.Cu") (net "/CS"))
 (segment (start 119.6848 35.8648) (end 125.5268 30.0228) (width 0.2) (layer "B.Cu") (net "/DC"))
 (segment (start 119.6848 35.8648) (end 109.1692 35.8648) (width 0.2) (layer "B.Cu") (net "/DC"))
 (segment (start 128.0668 30.0228) (end 119.6848 38.4048) (width 0.2) (layer "F.Cu") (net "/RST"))
 (segment (start 109.1692 38.4048) (end 119.6848 38.4048) (width 0.2) (layer "F.Cu") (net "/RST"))
 (segment (start 117.1448 43.4848) (end 109.1692 43.4848) (width 0.2) (layer "F.Cu") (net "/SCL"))
 (segment (start 117.1448 43.4848) (end 130.6068 30.0228) (width 0.2) (layer "F.Cu") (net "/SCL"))
 (segment (start 135.3312 55.0672) (end 135.6868 55.4228) (width 0.2) (layer "F.Cu") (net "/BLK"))
 (segment (start 131.7498 51.1302) (end 135.3312 54.7116) (width 0.2) (layer "F.Cu") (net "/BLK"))
 (segment (start 135.3312 54.7116) (end 135.3312 55.0672) (width 0.2) (layer "F.Cu") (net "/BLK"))
 (segment (start 115.8748 35.2552) (end 117.1448 36.5252) (width 0.2) (layer "F.Cu") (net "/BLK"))
 (via (at 115.8748 35.2552) (size 0.6) (drill 0.3) (layers "F.Cu" "B.Cu") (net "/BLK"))
 (via (at 131.7498 51.1302) (size 0.6) (drill 0.3) (layers "F.Cu" "B.Cu") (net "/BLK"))
 (via (at 117.1448 36.5252) (size 0.6) (drill 0.3) (layers "F.Cu" "B.Cu") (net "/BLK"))
 (segment (start 109.1692 30.7848) (end 113.6396 35.2552) (width 0.2) (layer "B.Cu") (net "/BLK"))
 (segment (start 131.7498 51.1302) (end 117.1448 36.5252) (width 0.2) (layer "B.Cu") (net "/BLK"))
 (segment (start 113.6396 35.2552) (end 115.8748 35.2552) (width 0.2) (layer "B.Cu") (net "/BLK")))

